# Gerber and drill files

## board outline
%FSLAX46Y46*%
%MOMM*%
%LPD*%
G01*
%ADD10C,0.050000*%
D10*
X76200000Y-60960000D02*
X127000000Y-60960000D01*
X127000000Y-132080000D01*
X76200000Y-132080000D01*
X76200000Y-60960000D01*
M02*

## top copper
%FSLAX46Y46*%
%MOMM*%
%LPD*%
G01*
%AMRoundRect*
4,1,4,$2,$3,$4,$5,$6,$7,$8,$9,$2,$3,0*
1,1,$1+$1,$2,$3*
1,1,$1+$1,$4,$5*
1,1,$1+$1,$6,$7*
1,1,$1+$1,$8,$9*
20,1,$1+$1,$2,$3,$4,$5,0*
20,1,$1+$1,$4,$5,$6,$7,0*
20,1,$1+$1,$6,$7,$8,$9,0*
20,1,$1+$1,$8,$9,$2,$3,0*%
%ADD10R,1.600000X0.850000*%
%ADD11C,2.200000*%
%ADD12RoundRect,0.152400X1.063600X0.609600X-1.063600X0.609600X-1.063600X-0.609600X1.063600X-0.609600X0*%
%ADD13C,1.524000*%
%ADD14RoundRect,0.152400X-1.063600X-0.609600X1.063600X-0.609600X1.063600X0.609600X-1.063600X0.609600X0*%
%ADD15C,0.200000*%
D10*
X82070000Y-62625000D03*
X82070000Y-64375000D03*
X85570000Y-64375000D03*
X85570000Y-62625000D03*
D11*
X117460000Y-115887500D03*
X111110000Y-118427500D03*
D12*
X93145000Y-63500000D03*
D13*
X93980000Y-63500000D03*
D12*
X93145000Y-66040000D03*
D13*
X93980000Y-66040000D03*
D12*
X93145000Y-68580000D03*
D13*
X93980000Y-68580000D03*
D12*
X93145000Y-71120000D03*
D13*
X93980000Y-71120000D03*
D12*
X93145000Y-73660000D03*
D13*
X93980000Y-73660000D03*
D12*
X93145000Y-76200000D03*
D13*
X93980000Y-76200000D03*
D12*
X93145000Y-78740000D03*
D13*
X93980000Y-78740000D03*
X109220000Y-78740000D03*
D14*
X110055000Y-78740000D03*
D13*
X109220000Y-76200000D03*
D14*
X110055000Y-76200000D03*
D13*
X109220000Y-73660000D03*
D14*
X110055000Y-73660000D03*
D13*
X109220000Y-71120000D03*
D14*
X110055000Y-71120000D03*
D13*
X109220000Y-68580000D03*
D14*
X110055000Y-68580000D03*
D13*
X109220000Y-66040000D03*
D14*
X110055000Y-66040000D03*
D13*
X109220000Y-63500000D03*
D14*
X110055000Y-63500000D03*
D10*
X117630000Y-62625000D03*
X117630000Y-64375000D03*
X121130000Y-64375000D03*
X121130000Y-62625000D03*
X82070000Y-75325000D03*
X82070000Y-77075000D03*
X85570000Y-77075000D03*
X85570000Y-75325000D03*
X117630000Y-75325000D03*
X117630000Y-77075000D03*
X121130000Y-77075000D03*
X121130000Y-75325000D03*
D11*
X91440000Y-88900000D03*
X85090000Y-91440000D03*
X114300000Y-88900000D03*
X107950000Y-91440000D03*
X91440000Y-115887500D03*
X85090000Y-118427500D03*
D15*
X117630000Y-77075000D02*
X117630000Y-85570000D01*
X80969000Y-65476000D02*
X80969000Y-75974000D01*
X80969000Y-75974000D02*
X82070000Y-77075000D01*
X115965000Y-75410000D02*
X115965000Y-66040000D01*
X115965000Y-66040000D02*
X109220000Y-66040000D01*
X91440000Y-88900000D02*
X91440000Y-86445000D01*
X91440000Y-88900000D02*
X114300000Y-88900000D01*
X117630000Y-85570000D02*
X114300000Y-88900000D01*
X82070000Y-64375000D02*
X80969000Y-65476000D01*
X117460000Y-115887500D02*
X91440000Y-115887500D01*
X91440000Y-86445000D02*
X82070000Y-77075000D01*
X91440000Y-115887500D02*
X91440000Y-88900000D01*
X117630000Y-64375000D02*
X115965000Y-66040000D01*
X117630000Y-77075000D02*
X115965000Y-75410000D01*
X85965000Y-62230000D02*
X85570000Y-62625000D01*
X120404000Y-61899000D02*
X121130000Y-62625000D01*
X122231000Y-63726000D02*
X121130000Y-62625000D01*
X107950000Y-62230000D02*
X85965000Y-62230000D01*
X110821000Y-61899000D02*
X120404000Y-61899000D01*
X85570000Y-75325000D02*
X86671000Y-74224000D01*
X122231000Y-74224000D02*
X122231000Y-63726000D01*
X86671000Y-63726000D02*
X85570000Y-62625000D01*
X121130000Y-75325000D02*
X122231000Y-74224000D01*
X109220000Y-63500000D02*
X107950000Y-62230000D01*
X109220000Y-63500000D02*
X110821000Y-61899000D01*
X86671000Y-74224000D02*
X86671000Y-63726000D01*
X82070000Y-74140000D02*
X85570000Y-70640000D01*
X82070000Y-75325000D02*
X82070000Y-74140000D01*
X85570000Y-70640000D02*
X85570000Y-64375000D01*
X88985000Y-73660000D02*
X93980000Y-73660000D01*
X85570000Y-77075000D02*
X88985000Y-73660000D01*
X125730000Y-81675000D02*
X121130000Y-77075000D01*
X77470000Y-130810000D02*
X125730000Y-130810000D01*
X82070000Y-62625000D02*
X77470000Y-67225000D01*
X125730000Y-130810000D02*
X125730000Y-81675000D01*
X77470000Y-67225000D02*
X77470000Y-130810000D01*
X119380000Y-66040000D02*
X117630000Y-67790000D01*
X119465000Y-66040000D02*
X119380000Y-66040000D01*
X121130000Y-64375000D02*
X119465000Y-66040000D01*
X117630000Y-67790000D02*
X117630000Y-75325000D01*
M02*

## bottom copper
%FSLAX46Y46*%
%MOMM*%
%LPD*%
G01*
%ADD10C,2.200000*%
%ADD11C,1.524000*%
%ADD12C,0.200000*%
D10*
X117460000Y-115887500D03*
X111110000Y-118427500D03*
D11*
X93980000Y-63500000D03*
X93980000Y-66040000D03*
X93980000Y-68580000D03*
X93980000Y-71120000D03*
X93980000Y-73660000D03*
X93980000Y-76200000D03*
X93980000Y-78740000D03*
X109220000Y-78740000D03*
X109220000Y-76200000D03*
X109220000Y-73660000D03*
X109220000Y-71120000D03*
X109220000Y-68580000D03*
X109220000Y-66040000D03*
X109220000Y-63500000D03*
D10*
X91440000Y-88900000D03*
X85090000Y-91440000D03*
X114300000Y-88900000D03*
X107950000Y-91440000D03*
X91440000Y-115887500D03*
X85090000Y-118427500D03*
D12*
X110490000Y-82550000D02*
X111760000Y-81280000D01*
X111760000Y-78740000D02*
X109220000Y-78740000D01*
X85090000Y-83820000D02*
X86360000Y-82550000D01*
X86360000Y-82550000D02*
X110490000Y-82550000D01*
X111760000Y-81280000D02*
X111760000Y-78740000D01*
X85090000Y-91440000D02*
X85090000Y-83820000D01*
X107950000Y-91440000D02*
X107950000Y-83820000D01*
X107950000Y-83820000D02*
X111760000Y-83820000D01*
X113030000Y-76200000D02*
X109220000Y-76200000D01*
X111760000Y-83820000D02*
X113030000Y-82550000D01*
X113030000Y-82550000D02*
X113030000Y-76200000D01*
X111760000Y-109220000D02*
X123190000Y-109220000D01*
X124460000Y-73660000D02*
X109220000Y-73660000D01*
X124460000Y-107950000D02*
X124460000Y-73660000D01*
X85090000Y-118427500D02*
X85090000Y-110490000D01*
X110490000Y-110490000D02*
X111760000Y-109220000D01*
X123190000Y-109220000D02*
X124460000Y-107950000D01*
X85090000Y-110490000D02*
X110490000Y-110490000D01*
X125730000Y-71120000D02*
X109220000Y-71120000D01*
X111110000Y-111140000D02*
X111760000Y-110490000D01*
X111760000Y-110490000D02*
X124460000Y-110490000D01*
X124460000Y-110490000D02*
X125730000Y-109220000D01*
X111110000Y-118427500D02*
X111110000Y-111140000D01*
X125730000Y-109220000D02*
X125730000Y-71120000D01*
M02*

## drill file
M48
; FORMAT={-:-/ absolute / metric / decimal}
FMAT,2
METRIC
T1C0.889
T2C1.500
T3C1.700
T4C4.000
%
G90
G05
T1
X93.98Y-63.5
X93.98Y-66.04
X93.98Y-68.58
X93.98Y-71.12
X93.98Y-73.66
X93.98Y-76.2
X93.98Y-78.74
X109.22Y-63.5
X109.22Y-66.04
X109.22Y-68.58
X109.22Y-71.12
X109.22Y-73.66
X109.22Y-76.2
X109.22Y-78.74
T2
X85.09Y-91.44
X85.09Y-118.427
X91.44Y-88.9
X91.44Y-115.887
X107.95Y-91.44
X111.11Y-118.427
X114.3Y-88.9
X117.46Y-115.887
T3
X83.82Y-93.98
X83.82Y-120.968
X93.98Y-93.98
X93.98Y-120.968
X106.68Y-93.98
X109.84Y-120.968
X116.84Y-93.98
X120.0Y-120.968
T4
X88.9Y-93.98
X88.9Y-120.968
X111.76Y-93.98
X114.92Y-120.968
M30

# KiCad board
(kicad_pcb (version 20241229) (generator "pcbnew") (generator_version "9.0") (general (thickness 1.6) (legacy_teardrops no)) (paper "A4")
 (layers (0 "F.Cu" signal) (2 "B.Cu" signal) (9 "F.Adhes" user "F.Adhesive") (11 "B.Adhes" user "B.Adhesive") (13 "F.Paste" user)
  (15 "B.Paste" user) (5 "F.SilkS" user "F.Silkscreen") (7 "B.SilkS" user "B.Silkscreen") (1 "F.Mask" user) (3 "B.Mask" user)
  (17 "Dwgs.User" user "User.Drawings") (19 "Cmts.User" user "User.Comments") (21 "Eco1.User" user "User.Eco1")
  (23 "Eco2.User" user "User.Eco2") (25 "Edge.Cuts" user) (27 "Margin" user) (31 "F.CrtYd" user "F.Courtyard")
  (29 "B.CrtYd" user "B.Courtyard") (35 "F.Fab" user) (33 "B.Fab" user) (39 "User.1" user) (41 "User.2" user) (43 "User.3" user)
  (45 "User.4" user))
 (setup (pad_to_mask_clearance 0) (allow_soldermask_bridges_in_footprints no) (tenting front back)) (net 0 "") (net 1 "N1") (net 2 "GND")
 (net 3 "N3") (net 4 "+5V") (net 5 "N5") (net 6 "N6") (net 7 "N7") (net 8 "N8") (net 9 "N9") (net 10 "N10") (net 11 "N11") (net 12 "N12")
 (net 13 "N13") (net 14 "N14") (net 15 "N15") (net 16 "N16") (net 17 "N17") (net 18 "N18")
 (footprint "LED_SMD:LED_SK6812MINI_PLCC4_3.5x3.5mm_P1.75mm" (layer "F.Cu") (at 83.82 63.5)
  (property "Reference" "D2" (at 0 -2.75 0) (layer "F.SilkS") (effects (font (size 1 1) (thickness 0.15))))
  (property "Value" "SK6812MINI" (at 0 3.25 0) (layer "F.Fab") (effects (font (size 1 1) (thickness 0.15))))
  (pad "1" smd rect (at -1.75 -0.875) (size 1.6 0.85) (layers "F.Cu" "F.Mask" "F.Paste") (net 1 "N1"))
  (pad "2" smd rect (at -1.75 0.875) (size 1.6 0.85) (layers "F.Cu" "F.Mask" "F.Paste") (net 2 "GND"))
  (pad "3" smd rect (at 1.75 0.875) (size 1.6 0.85) (layers "F.Cu" "F.Mask" "F.Paste") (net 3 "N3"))
  (pad "4" smd rect (at 1.75 -0.875) (size 1.6 0.85) (layers "F.Cu" "F.Mask" "F.Paste") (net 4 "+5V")))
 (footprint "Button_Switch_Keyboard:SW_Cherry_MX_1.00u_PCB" (layer "F.Cu") (at 117.46 115.8875)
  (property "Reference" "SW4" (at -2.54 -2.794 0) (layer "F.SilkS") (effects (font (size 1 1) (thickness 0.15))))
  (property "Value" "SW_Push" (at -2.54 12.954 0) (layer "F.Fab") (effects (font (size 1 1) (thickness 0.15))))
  (pad "" np_thru_hole circle (at -7.62 5.08) (size 1.7 1.7) (drill 1.7) (layers "*.Cu" "*.Mask"))
  (pad "" np_thru_hole circle (at -2.54 5.08) (size 4 4) (drill 4) (layers "*.Cu" "*.Mask"))
  (pad "" np_thru_hole circle (at 2.54 5.08) (size 1.7 1.7) (drill 1.7) (layers "*.Cu" "*.Mask"))
  (pad "1" thru_hole circle (at 0 0) (size 2.2 2.2) (drill 1.5) (layers "*.Cu" "*.Mask") (remove_unused_layers no) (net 2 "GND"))
  (pad "2" thru_hole circle (at -6.35 2.54) (size 2.2 2.2) (drill 1.5) (layers "*.Cu" "*.Mask") (remove_unused_layers no) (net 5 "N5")))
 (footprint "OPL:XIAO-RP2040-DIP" (layer "F.Cu") (at 101.6 71.12)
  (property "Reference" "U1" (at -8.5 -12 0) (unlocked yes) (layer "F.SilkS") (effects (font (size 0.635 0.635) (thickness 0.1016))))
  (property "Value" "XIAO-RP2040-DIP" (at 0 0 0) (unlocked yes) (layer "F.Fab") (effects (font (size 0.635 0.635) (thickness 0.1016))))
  (pad "1" smd roundrect (at -8.455 -7.62 180) (size 2.432 1.524) (layers "F.Cu" "F.Mask") (roundrect_rratio 0.1) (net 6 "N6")
   (thermal_bridge_angle 45))
  (pad "1" thru_hole circle (at -7.62 -7.62 180) (size 1.524 1.524) (drill 0.889) (layers "*.Cu" "*.Mask") (remove_unused_layers no)
   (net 6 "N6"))
  (pad "2" smd roundrect (at -8.455 -5.08 180) (size 2.432 1.524) (layers "F.Cu" "F.Mask") (roundrect_rratio 0.1) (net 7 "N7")
   (thermal_bridge_angle 45))
  (pad "2" thru_hole circle (at -7.62 -5.08 180) (size 1.524 1.524) (drill 0.889) (layers "*.Cu" "*.Mask") (remove_unused_layers no)
   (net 7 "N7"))
  (pad "3" smd roundrect (at -8.455 -2.54 180) (size 2.432 1.524) (layers "F.Cu" "F.Mask") (roundrect_rratio 0.1) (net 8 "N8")
   (thermal_bridge_angle 45))
  (pad "3" thru_hole circle (at -7.62 -2.54 180) (size 1.524 1.524) (drill 0.889) (layers "*.Cu" "*.Mask") (remove_unused_layers no)
   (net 8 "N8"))
  (pad "4" smd roundrect (at -8.455 0 180) (size 2.432 1.524) (layers "F.Cu" "F.Mask") (roundrect_rratio 0.1) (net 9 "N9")
   (thermal_bridge_angle 45))
  (pad "4" thru_hole circle (at -7.62 0 180) (size 1.524 1.524) (drill 0.889) (layers "*.Cu" "*.Mask") (remove_unused_layers no)
   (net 9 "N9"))
  (pad "5" smd roundrect (at -8.455 2.54 180) (size 2.432 1.524) (layers "F.Cu" "F.Mask") (roundrect_rratio 0.1) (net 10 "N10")
   (thermal_bridge_angle 45))
  (pad "5" thru_hole circle (at -7.62 2.54 180) (size 1.524 1.524) (drill 0.889) (layers "*.Cu" "*.Mask") (remove_unused_layers no)
   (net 10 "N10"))
  (pad "6" smd roundrect (at -8.455 5.08 180) (size 2.432 1.524) (layers "F.Cu" "F.Mask") (roundrect_rratio 0.1) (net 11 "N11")
   (thermal_bridge_angle 45))
  (pad "6" thru_hole circle (at -7.62 5.08 180) (size 1.524 1.524) (drill 0.889) (layers "*.Cu" "*.Mask") (remove_unused_layers no)
   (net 11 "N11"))
  (pad "7" smd roundrect (at -8.455 7.62 180) (size 2.432 1.524) (layers "F.Cu" "F.Mask") (roundrect_rratio 0.1) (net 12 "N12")
   (thermal_bridge_angle 45))
  (pad "7" thru_hole circle (at -7.62 7.62 180) (size 1.524 1.524) (drill 0.889) (layers "*.Cu" "*.Mask") (remove_unused_layers no)
   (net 12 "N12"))
  (pad "8" thru_hole circle (at 7.62 7.62) (size 1.524 1.524) (drill 0.889) (layers "*.Cu" "*.Mask") (remove_unused_layers no)
   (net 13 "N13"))
  (pad "8" smd roundrect (at 8.455 7.62) (size 2.432 1.524) (layers "F.Cu" "F.Mask") (roundrect_rratio 0.1) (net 13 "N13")
   (thermal_bridge_angle 45))
  (pad "9" thru_hole circle (at 7.62 5.08) (size 1.524 1.524) (drill 0.889) (layers "*.Cu" "*.Mask") (remove_unused_layers no)
   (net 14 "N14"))
  (pad "9" smd roundrect (at 8.455 5.08) (size 2.432 1.524) (layers "F.Cu" "F.Mask") (roundrect_rratio 0.1) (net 14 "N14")
   (thermal_bridge_angle 45))
  (pad "10" thru_hole circle (at 7.62 2.54) (size 1.524 1.524) (drill 0.889) (layers "*.Cu" "*.Mask") (remove_unused_layers no)
   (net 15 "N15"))
  (pad "10" smd roundrect (at 8.455 2.54) (size 2.432 1.524) (layers "F.Cu" "F.Mask") (roundrect_rratio 0.1) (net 15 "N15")
   (thermal_bridge_angle 45))
  (pad "11" thru_hole circle (at 7.62 0) (size 1.524 1.524) (drill 0.889) (layers "*.Cu" "*.Mask") (remove_unused_layers no) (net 5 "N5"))
  (pad "11" smd roundrect (at 8.455 0) (size 2.432 1.524) (layers "F.Cu" "F.Mask") (roundrect_rratio 0.1) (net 5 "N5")
   (thermal_bridge_angle 45))
  (pad "12" thru_hole circle (at 7.62 -2.54) (size 1.524 1.524) (drill 0.889) (layers "*.Cu" "*.Mask") (remove_unused_layers no)
   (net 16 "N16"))
  (pad "12" smd roundrect (at 8.455 -2.54) (size 2.432 1.524) (layers "F.Cu" "F.Mask") (roundrect_rratio 0.1) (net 16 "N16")
   (thermal_bridge_angle 45))
  (pad "13" thru_hole circle (at 7.62 -5.08) (size 1.524 1.524) (drill 0.889) (layers "*.Cu" "*.Mask") (remove_unused_layers no)
   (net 2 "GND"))
  (pad "13" smd roundrect (at 8.455 -5.08) (size 2.432 1.524) (layers "F.Cu" "F.Mask") (roundrect_rratio 0.1) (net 2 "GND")
   (thermal_bridge_angle 45))
  (pad "14" thru_hole circle (at 7.62 -7.62) (size 1.524 1.524) (drill 0.889) (layers "*.Cu" "*.Mask") (remove_unused_layers no)
   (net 4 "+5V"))
  (pad "14" smd roundrect (at 8.455 -7.62) (size 2.432 1.524) (layers "F.Cu" "F.Mask") (roundrect_rratio 0.1) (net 4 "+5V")
   (thermal_bridge_angle 45)))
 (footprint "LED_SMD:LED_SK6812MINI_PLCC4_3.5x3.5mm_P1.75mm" (layer "F.Cu") (at 119.38 63.5)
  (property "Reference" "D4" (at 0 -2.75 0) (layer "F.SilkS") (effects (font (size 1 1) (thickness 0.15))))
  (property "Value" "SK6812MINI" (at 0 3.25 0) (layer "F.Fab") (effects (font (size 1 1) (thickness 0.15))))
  (pad "1" smd rect (at -1.75 -0.875) (size 1.6 0.85) (layers "F.Cu" "F.Mask" "F.Paste") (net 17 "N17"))
  (pad "2" smd rect (at -1.75 0.875) (size 1.6 0.85) (layers "F.Cu" "F.Mask" "F.Paste") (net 2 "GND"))
  (pad "3" smd rect (at 1.75 0.875) (size 1.6 0.85) (layers "F.Cu" "F.Mask" "F.Paste") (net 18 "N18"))
  (pad "4" smd rect (at 1.75 -0.875) (size 1.6 0.85) (layers "F.Cu" "F.Mask" "F.Paste") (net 4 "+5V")))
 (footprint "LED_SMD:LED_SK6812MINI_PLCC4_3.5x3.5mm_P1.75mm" (layer "F.Cu") (at 83.82 76.2)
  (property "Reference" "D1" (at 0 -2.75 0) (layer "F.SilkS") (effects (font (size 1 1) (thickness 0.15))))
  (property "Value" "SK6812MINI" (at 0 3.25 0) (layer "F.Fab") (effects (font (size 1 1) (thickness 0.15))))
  (pad "1" smd rect (at -1.75 -0.875) (size 1.6 0.85) (layers "F.Cu" "F.Mask" "F.Paste") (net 3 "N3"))
  (pad "2" smd rect (at -1.75 0.875) (size 1.6 0.85) (layers "F.Cu" "F.Mask" "F.Paste") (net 2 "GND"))
  (pad "3" smd rect (at 1.75 0.875) (size 1.6 0.85) (layers "F.Cu" "F.Mask" "F.Paste") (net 10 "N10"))
  (pad "4" smd rect (at 1.75 -0.875) (size 1.6 0.85) (layers "F.Cu" "F.Mask" "F.Paste") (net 4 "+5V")))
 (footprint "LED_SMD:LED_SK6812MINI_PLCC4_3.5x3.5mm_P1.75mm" (layer "F.Cu") (at 119.38 76.2)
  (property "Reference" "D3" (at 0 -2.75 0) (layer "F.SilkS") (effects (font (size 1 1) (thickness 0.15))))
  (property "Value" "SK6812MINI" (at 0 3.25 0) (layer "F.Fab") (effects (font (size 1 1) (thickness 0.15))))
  (pad "1" smd rect (at -1.75 -0.875) (size 1.6 0.85) (layers "F.Cu" "F.Mask" "F.Paste") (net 18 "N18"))
  (pad "2" smd rect (at -1.75 0.875) (size 1.6 0.85) (layers "F.Cu" "F.Mask" "F.Paste") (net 2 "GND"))
  (pad "3" smd rect (at 1.75 0.875) (size 1.6 0.85) (layers "F.Cu" "F.Mask" "F.Paste") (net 1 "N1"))
  (pad "4" smd rect (at 1.75 -0.875) (size 1.6 0.85) (layers "F.Cu" "F.Mask" "F.Paste") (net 4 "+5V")))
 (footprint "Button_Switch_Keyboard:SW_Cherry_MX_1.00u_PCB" (layer "F.Cu") (at 91.44 88.9)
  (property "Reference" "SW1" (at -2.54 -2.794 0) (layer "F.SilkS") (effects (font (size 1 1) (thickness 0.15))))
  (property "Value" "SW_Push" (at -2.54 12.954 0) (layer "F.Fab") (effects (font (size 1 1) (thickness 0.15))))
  (pad "" np_thru_hole circle (at -7.62 5.08) (size 1.7 1.7) (drill 1.7) (layers "*.Cu" "*.Mask"))
  (pad "" np_thru_hole circle (at -2.54 5.08) (size 4 4) (drill 4) (layers "*.Cu" "*.Mask"))
  (pad "" np_thru_hole circle (at 2.54 5.08) (size 1.7 1.7) (drill 1.7) (layers "*.Cu" "*.Mask"))
  (pad "1" thru_hole circle (at 0 0) (size 2.2 2.2) (drill 1.5) (layers "*.Cu" "*.Mask") (remove_unused_layers no) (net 2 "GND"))
  (pad "2" thru_hole circle (at -6.35 2.54) (size 2.2 2.2) (drill 1.5) (layers "*.Cu" "*.Mask") (remove_unused_layers no) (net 13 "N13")))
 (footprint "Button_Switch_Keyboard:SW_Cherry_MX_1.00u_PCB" (layer "F.Cu") (at 114.3 88.9)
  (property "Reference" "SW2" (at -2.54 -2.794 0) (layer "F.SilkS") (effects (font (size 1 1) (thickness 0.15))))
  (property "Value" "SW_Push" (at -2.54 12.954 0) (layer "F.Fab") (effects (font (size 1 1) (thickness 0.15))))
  (pad "" np_thru_hole circle (at -7.62 5.08) (size 1.7 1.7) (drill 1.7) (layers "*.Cu" "*.Mask"))
  (pad "" np_thru_hole circle (at -2.54 5.08) (size 4 4) (drill 4) (layers "*.Cu" "*.Mask"))
  (pad "" np_thru_hole circle (at 2.54 5.08) (size 1.7 1.7) (drill 1.7) (layers "*.Cu" "*.Mask"))
  (pad "1" thru_hole circle (at 0 0) (size 2.2 2.2) (drill 1.5) (layers "*.Cu" "*.Mask") (remove_unused_layers no) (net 2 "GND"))
  (pad "2" thru_hole circle (at -6.35 2.54) (size 2.2 2.2) (drill 1.5) (layers "*.Cu" "*.Mask") (remove_unused_layers no) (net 14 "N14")))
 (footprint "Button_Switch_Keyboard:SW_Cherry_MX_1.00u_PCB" (layer "F.Cu") (at 91.44 115.8875)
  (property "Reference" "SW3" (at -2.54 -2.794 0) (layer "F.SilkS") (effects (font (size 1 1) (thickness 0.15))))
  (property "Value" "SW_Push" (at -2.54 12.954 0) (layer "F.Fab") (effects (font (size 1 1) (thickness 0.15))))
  (pad "" np_thru_hole circle (at -7.62 5.08) (size 1.7 1.7) (drill 1.7) (layers "*.Cu" "*.Mask"))
  (pad "" np_thru_hole circle (at -2.54 5.08) (size 4 4) (drill 4) (layers "*.Cu" "*.Mask"))
  (pad "" np_thru_hole circle (at 2.54 5.08) (size 1.7 1.7) (drill 1.7) (layers "*.Cu" "*.Mask"))
  (pad "1" thru_hole circle (at 0 0) (size 2.2 2.2) (drill 1.5) (layers "*.Cu" "*.Mask") (remove_unused_layers no) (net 2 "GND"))
  (pad "2" thru_hole circle (at -6.35 2.54) (size 2.2 2.2) (drill 1.5) (layers "*.Cu" "*.Mask") (remove_unused_layers no) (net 15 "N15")))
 (gr_rect (start 76.2 60.96) (end 127 132.08) (stroke (width 0.05) (type default)) (fill no) (layer "Edge.Cuts"))
 (segment (start 117.63 77.075) (end 117.63 85.57) (width 0.2) (layer "F.Cu") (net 2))
 (segment (start 80.969 65.476) (end 80.969 75.974) (width 0.2) (layer "F.Cu") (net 2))
 (segment (start 80.969 75.974) (end 82.07 77.075) (width 0.2) (layer "F.Cu") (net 2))
 (segment (start 115.965 75.41) (end 115.965 66.04) (width 0.2) (layer "F.Cu") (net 2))
 (segment (start 115.965 66.04) (end 109.22 66.04) (width 0.2) (layer "F.Cu") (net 2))
 (segment (start 91.44 88.9) (end 91.44 86.445) (width 0.2) (layer "F.Cu") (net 2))
 (segment (start 91.44 88.9) (end 114.3 88.9) (width 0.2) (layer "F.Cu") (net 2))
 (segment (start 117.63 85.57) (end 114.3 88.9) (width 0.2) (layer "F.Cu") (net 2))
 (segment (start 82.07 64.375) (end 80.969 65.476) (width 0.2) (layer "F.Cu") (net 2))
 (segment (start 117.46 115.8875) (end 91.44 115.8875) (width 0.2) (layer "F.Cu") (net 2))
 (segment (start 91.44 86.445) (end 82.07 77.075) (width 0.2) (layer "F.Cu") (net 2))
 (segment (start 91.44 115.8875) (end 91.44 88.9) (width 0.2) (layer "F.Cu") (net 2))
 (segment (start 117.63 64.375) (end 115.965 66.04) (width 0.2) (layer "F.Cu") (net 2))
 (segment (start 117.63 77.075) (end 115.965 75.41) (width 0.2) (layer "F.Cu") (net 2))
 (segment (start 85.965 62.23) (end 85.57 62.625) (width 0.2) (layer "F.Cu") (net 4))
 (segment (start 120.404 61.899) (end 121.13 62.625) (width 0.2) (layer "F.Cu") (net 4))
 (segment (start 122.231 63.726) (end 121.13 62.625) (width 0.2) (layer "F.Cu") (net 4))
 (segment (start 107.95 62.23) (end 85.965 62.23) (width 0.2) (layer "F.Cu") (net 4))
 (segment (start 110.821 61.899) (end 120.404 61.899) (width 0.2) (layer "F.Cu") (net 4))
 (segment (start 85.57 75.325) (end 86.671 74.224) (width 0.2) (layer "F.Cu") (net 4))
 (segment (start 122.231 74.224) (end 122.231 63.726) (width 0.2) (layer "F.Cu") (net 4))
 (segment (start 86.671 63.726) (end 85.57 62.625) (width 0.2) (layer "F.Cu") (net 4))
 (segment (start 121.13 75.325) (end 122.231 74.224) (width 0.2) (layer "F.Cu") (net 4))
 (segment (start 109.22 63.5) (end 107.95 62.23) (width 0.2) (layer "F.Cu") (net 4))
 (segment (start 109.22 63.5) (end 110.821 61.899) (width 0.2) (layer "F.Cu") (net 4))
 (segment (start 86.671 74.224) (end 86.671 63.726) (width 0.2) (layer "F.Cu") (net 4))
 (segment (start 82.07 74.14) (end 85.57 70.64) (width 0.2) (layer "F.Cu") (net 3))
 (segment (start 82.07 75.325) (end 82.07 74.14) (width 0.2) (layer "F.Cu") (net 3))
 (segment (start 85.57 70.64) (end 85.57 64.375) (width 0.2) (layer "F.Cu") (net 3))
 (segment (start 88.985 73.66) (end 93.98 73.66) (width 0.2) (layer "F.Cu") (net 10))
 (segment (start 85.57 77.075) (end 88.985 73.66) (width 0.2) (layer "F.Cu") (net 10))
 (segment (start 125.73 81.675) (end 121.13 77.075) (width 0.2) (layer "F.Cu") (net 1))
 (segment (start 77.47 130.81) (end 125.73 130.81) (width 0.2) (layer "F.Cu") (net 1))
 (segment (start 82.07 62.625) (end 77.47 67.225) (width 0.2) (layer "F.Cu") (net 1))
 (segment (start 125.73 130.81) (end 125.73 81.675) (width 0.2) (layer "F.Cu") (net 1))
 (segment (start 77.47 67.225) (end 77.47 130.81) (width 0.2) (layer "F.Cu") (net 1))
 (segment (start 119.38 66.04) (end 117.63 67.79) (width 0.2) (layer "F.Cu") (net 18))
 (segment (start 119.465 66.04) (end 119.38 66.04) (width 0.2) (layer "F.Cu") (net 18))
 (segment (start 121.13 64.375) (end 119.465 66.04) (width 0.2) (layer "F.Cu") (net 18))
 (segment (start 117.63 67.79) (end 117.63 75.325) (width 0.2) (layer "F.Cu") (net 18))
 (segment (start 110.49 82.55) (end 111.76 81.28) (width 0.2) (layer "B.Cu") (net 13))
 (segment (start 111.76 78.74) (end 109.22 78.74) (width 0.2) (layer "B.Cu") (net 13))
 (segment (start 85.09 83.82) (end 86.36 82.55) (width 0.2) (layer "B.Cu") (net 13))
 (segment (start 86.36 82.55) (end 110.49 82.55) (width 0.2) (layer "B.Cu") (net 13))
 (segment (start 111.76 81.28) (end 111.76 78.74) (width 0.2) (layer "B.Cu") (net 13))
 (segment (start 85.09 91.44) (end 85.09 83.82) (width 0.2) (layer "B.Cu") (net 13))
 (segment (start 107.95 91.44) (end 107.95 83.82) (width 0.2) (layer "B.Cu") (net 14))
 (segment (start 107.95 83.82) (end 111.76 83.82) (width 0.2) (layer "B.Cu") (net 14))
 (segment (start 113.03 76.2) (end 109.22 76.2) (width 0.2) (layer "B.Cu") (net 14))
 (segment (start 111.76 83.82) (end 113.03 82.55) (width 0.2) (layer "B.Cu") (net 14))
 (segment (start 113.03 82.55) (end 113.03 76.2) (width 0.2) (layer "B.Cu") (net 14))
 (segment (start 111.76 109.22) (end 123.19 109.22) (width 0.2) (layer "B.Cu") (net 15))
 (segment (start 124.46 73.66) (end 109.22 73.66) (width 0.2) (layer "B.Cu") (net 15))
 (segment (start 124.46 107.95) (end 124.46 73.66) (width 0.2) (layer "B.Cu") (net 15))
 (segment (start 85.09 118.4275) (end 85.09 110.49) (width 0.2) (layer "B.Cu") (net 15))
 (segment (start 110.49 110.49) (end 111.76 109.22) (width 0.2) (layer "B.Cu") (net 15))
 (segment (start 123.19 109.22) (end 124.46 107.95) (width 0.2) (layer "B.Cu") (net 15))
 (segment (start 85.09 110.49) (end 110.49 110.49) (width 0.2) (layer "B.Cu") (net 15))
 (segment (start 125.73 71.12) (end 109.22 71.12) (width 0.2) (layer "B.Cu") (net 5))
 (segment (start 111.11 111.14) (end 111.76 110.49) (width 0.2) (layer "B.Cu") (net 5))
 (segment (start 111.76 110.49) (end 124.46 110.49) (width 0.2) (layer "B.Cu") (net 5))
 (segment (start 124.46 110.49) (end 125.73 109.22) (width 0.2) (layer "B.Cu") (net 5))
 (segment (start 111.11 118.4275) (end 111.11 111.14) (width 0.2) (layer "B.Cu") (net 5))
 (segment (start 125.73 109.22) (end 125.73 71.12) (width 0.2) (layer "B.Cu") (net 5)))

